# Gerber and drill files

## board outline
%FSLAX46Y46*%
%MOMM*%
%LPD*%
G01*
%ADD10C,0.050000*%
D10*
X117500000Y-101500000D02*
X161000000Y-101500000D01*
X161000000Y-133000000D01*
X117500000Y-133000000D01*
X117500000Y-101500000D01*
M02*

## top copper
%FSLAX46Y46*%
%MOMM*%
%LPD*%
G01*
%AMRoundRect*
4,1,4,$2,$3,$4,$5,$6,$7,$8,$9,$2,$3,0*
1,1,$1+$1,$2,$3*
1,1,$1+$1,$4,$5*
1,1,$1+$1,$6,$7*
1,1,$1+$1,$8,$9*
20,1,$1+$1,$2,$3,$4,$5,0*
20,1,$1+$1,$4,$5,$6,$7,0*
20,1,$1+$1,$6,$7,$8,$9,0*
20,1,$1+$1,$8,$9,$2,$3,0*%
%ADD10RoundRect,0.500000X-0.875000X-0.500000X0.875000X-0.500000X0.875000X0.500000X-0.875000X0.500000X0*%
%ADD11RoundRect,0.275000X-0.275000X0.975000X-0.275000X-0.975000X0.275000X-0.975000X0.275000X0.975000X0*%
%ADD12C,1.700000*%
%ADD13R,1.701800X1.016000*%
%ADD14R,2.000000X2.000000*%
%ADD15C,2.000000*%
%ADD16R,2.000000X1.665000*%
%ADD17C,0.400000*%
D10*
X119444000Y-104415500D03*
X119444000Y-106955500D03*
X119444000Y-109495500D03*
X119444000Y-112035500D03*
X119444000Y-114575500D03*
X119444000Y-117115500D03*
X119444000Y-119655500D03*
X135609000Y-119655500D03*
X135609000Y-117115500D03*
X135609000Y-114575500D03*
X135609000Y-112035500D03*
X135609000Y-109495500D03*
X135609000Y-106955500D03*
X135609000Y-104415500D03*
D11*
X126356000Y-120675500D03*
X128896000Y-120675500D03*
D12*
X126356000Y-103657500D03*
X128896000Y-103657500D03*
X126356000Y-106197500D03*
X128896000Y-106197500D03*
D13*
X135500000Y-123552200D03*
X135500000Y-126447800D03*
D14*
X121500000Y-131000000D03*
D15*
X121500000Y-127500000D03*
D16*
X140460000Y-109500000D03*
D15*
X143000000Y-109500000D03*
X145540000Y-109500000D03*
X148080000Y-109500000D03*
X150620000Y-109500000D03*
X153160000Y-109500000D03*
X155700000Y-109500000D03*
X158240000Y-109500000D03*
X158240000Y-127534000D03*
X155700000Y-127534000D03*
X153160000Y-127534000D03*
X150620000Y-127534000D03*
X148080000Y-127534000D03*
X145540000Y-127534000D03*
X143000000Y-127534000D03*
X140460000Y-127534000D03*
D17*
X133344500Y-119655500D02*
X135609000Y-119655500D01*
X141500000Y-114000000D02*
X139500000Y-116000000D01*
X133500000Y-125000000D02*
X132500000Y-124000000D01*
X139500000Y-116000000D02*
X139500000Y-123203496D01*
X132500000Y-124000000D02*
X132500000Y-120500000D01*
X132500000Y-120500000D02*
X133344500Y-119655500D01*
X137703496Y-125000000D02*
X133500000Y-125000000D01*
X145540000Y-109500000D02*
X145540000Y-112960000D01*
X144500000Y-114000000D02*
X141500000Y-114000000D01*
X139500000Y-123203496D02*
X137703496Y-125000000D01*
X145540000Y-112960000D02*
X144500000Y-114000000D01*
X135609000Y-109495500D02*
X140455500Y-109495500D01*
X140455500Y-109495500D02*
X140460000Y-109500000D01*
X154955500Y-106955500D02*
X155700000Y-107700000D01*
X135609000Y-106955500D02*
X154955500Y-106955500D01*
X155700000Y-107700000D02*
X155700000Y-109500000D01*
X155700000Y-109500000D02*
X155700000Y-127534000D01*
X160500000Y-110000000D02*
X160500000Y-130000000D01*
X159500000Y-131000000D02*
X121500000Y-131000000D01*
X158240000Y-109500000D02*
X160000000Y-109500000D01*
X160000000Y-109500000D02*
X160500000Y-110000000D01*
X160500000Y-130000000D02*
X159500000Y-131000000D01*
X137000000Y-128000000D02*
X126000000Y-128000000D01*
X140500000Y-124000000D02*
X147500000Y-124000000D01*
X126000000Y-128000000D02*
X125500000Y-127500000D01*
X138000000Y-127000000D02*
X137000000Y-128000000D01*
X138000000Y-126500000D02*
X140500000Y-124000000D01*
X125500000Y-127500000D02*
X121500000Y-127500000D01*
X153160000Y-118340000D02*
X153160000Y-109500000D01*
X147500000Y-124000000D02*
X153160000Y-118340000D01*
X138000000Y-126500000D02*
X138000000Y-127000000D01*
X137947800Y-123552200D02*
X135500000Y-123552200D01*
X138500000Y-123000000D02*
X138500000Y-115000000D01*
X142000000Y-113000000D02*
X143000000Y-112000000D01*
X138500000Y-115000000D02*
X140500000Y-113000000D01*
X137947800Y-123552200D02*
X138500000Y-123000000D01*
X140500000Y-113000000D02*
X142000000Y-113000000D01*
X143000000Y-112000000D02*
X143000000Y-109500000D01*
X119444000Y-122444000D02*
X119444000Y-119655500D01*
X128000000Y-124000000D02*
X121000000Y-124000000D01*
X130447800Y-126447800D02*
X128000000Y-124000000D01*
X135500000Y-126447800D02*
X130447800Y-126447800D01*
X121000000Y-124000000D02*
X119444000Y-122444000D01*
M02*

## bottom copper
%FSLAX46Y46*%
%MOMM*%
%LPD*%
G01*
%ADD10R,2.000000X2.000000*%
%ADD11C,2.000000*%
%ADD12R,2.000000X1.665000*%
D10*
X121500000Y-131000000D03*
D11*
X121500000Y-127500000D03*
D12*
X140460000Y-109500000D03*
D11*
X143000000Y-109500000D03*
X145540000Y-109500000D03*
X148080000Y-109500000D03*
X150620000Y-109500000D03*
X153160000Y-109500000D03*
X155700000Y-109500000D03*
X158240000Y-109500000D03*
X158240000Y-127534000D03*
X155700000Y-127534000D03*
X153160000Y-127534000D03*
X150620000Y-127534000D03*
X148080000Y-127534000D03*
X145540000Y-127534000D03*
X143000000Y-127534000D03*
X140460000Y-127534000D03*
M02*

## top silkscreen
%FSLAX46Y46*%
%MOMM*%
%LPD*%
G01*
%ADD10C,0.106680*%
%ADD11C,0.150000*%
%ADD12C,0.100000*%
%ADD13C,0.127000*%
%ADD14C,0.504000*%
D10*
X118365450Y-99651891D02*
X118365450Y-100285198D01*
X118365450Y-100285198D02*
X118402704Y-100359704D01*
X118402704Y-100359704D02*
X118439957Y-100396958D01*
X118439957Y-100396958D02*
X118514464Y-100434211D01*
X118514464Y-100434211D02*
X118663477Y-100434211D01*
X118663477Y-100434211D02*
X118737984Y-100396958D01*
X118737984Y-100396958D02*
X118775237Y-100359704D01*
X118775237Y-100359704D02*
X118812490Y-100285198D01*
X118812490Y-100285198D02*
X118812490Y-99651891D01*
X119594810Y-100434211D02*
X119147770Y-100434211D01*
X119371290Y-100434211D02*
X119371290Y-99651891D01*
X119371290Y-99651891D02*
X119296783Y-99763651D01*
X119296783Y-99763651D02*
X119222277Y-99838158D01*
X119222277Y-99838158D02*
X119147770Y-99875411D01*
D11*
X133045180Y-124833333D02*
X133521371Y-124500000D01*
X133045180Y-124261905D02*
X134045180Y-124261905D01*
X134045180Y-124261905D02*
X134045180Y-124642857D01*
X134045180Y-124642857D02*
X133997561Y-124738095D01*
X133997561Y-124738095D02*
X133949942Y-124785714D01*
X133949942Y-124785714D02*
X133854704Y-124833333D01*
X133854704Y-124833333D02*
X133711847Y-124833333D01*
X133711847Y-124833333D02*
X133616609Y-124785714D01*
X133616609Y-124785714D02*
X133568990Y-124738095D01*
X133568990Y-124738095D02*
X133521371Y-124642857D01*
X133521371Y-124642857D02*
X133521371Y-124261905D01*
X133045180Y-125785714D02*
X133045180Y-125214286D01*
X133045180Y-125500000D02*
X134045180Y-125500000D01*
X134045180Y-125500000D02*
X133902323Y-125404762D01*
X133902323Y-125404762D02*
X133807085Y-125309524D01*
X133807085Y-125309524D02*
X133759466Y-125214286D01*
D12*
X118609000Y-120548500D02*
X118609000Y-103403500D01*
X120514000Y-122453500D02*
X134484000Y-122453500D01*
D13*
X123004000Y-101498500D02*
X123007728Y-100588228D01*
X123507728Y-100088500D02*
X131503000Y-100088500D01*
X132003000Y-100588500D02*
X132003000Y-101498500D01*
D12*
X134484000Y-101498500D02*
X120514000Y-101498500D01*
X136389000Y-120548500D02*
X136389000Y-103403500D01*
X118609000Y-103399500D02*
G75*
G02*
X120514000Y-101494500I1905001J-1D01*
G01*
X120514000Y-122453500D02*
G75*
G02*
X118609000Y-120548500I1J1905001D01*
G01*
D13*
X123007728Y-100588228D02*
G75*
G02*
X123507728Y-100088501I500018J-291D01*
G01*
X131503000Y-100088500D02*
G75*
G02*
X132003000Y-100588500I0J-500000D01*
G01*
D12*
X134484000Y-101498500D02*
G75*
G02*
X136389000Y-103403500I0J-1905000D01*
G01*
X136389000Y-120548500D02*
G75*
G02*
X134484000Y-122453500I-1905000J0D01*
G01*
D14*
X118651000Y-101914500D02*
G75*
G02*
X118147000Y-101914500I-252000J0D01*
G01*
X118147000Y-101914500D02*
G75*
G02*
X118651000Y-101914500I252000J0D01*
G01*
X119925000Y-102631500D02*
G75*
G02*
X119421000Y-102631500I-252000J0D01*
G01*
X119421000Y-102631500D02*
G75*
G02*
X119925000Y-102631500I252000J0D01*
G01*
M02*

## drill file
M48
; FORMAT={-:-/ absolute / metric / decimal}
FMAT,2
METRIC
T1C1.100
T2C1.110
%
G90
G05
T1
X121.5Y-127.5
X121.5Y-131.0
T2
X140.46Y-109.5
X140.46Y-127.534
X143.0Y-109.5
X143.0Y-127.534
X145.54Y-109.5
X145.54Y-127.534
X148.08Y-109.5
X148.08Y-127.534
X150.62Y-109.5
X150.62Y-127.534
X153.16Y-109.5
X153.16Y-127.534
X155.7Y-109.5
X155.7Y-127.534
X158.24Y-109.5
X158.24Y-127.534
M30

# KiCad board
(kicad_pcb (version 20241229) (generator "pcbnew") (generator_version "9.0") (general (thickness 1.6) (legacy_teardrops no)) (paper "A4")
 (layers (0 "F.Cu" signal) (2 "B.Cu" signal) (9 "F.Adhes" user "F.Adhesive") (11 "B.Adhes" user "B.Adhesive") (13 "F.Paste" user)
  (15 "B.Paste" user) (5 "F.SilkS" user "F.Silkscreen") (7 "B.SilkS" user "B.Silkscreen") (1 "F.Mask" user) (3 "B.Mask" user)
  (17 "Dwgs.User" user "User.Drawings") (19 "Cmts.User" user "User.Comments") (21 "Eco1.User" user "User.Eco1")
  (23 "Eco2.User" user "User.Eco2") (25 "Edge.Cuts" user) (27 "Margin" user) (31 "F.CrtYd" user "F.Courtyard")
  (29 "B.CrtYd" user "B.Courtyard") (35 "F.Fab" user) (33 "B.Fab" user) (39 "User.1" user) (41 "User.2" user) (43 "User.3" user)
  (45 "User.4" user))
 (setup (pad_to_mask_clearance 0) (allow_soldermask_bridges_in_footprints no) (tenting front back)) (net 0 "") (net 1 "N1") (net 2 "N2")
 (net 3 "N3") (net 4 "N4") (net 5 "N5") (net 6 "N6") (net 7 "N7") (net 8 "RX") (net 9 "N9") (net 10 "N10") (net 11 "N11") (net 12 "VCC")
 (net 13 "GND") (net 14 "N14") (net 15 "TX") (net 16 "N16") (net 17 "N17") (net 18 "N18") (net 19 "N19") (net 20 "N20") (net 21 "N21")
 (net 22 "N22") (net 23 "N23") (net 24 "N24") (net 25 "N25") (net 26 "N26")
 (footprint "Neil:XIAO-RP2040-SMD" (layer "F.Cu") (at 127.444 112.0355)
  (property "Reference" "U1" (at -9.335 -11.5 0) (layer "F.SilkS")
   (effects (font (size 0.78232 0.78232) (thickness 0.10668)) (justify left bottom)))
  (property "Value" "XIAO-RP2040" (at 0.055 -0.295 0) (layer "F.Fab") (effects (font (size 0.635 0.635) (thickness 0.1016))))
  (fp_line (start -8.835 8.513) (end -8.835 -8.632) (stroke (width 0.1) (type solid)) (layer "F.SilkS"))
  (fp_line (start -6.93 10.418) (end 7.04 10.418) (stroke (width 0.1) (type solid)) (layer "F.SilkS"))
  (fp_line (start -4.44 -10.537) (end -4.436272 -11.447272) (stroke (width 0.127) (type solid)) (layer "F.SilkS"))
  (fp_line (start -3.936272 -11.947) (end 4.059 -11.947) (stroke (width 0.127) (type solid)) (layer "F.SilkS"))
  (fp_line (start 4.559 -11.447) (end 4.559 -10.537) (stroke (width 0.127) (type solid)) (layer "F.SilkS"))
  (fp_line (start 7.04 -10.537) (end -6.93 -10.537) (stroke (width 0.1) (type solid)) (layer "F.SilkS"))
  (fp_line (start 8.945 8.513) (end 8.945 -8.632) (stroke (width 0.1) (type solid)) (layer "F.SilkS"))
  (fp_arc (start -8.835 -8.636) (mid -8.277038 -9.983038) (end -6.93 -10.541) (stroke (width 0.1) (type solid)) (layer "F.SilkS"))
  (fp_arc (start -6.93 10.418) (mid -8.277038 9.860038) (end -8.835 8.513) (stroke (width 0.1) (type solid)) (layer "F.SilkS"))
  (fp_arc (start -4.436272 -11.447272) (mid -4.289724 -11.800644) (end -3.936272 -11.947) (stroke (width 0.127) (type default))
   (layer "F.SilkS"))
  (fp_arc (start 4.059 -11.947) (mid 4.412553 -11.800553) (end 4.559 -11.447) (stroke (width 0.127) (type default)) (layer "F.SilkS"))
  (fp_arc (start 7.04 -10.537) (mid 8.387038 -9.979038) (end 8.945 -8.632) (stroke (width 0.1) (type solid)) (layer "F.SilkS"))
  (fp_arc (start 8.945 8.513) (mid 8.387038 9.860038) (end 7.04 10.418) (stroke (width 0.1) (type solid)) (layer "F.SilkS"))
  (fp_circle (center -9.045 -10.121) (end -9.045 -10.375) (stroke (width 0.5) (type solid)) (fill yes) (layer "F.SilkS"))
  (fp_circle (center -7.771 -9.404) (end -7.771 -9.658) (stroke (width 0.5) (type solid)) (fill yes) (layer "F.SilkS"))
  (pad "1" smd roundrect (at -8 -7.62) (size 2.75 2) (layers "F.Cu" "F.Mask" "F.Paste") (roundrect_rratio 0.25) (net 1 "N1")
   (solder_mask_margin 0.0508) (thermal_bridge_angle 45))
  (pad "2" smd roundrect (at -8 -5.08) (size 2.75 2) (layers "F.Cu" "F.Mask" "F.Paste") (roundrect_rratio 0.25) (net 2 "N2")
   (solder_mask_margin 0.0508) (thermal_bridge_angle 45))
  (pad "3" smd roundrect (at -8 -2.54) (size 2.75 2) (layers "F.Cu" "F.Mask" "F.Paste") (roundrect_rratio 0.25) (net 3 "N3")
   (solder_mask_margin 0.0508) (thermal_bridge_angle 45))
  (pad "4" smd roundrect (at -8 0) (size 2.75 2) (layers "F.Cu" "F.Mask" "F.Paste") (roundrect_rratio 0.25) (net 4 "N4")
   (solder_mask_margin 0.0508) (thermal_bridge_angle 45))
  (pad "5" smd roundrect (at -8 2.54) (size 2.75 2) (layers "F.Cu" "F.Mask" "F.Paste") (roundrect_rratio 0.25) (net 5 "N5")
   (solder_mask_margin 0.0508) (thermal_bridge_angle 45))
  (pad "6" smd roundrect (at -8 5.08) (size 2.75 2) (layers "F.Cu" "F.Mask" "F.Paste") (roundrect_rratio 0.25) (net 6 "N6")
   (solder_mask_margin 0.0508) (thermal_bridge_angle 45))
  (pad "7" smd roundrect (at -8 7.62) (size 2.75 2) (layers "F.Cu" "F.Mask" "F.Paste") (roundrect_rratio 0.25) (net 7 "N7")
   (solder_mask_margin 0.0508) (thermal_bridge_angle 45))
  (pad "8" smd roundrect (at 8.165 7.62) (size 2.75 2) (layers "F.Cu" "F.Mask" "F.Paste") (roundrect_rratio 0.25) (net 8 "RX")
   (solder_mask_margin 0.0508) (thermal_bridge_angle 45))
  (pad "9" smd roundrect (at 8.165 5.08) (size 2.75 2) (layers "F.Cu" "F.Mask" "F.Paste") (roundrect_rratio 0.25) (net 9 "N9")
   (solder_mask_margin 0.0508) (thermal_bridge_angle 45))
  (pad "10" smd roundrect (at 8.165 2.54) (size 2.75 2) (layers "F.Cu" "F.Mask" "F.Paste") (roundrect_rratio 0.25) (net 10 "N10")
   (solder_mask_margin 0.0508) (thermal_bridge_angle 45))
  (pad "11" smd roundrect (at 8.165 0) (size 2.75 2) (layers "F.Cu" "F.Mask" "F.Paste") (roundrect_rratio 0.25) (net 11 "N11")
   (solder_mask_margin 0.0508) (thermal_bridge_angle 45))
  (pad "12" smd roundrect (at 8.165 -2.54) (size 2.75 2) (layers "F.Cu" "F.Mask" "F.Paste") (roundrect_rratio 0.25) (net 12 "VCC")
   (solder_mask_margin 0.0508) (thermal_bridge_angle 45))
  (pad "13" smd roundrect (at 8.165 -5.08) (size 2.75 2) (layers "F.Cu" "F.Mask" "F.Paste") (roundrect_rratio 0.25) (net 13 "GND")
   (solder_mask_margin 0.0508) (thermal_bridge_angle 45))
  (pad "14" smd roundrect (at 8.165 -7.62) (size 2.75 2) (layers "F.Cu" "F.Mask" "F.Paste") (roundrect_rratio 0.25) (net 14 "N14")
   (solder_mask_margin 0.0508) (thermal_bridge_angle 45))
  (pad "15" smd roundrect (at -1.088 8.64 270) (size 2.5 1.1) (layers "F.Cu" "F.Mask" "F.Paste") (roundrect_rratio 0.25)
   (thermal_bridge_angle 45))
  (pad "16" smd roundrect (at 1.452 8.64 270) (size 2.5 1.1) (layers "F.Cu" "F.Mask" "F.Paste") (roundrect_rratio 0.25)
   (thermal_bridge_angle 45))
  (pad "17" smd circle (at -1.088 -8.378) (size 1.7 1.7) (layers "F.Cu" "F.Mask" "F.Paste"))
  (pad "18" smd circle (at 1.452 -8.378) (size 1.7 1.7) (layers "F.Cu" "F.Mask" "F.Paste"))
  (pad "19" smd circle (at -1.088 -5.838) (size 1.7 1.7) (layers "F.Cu" "F.Mask" "F.Paste"))
  (pad "20" smd circle (at 1.452 -5.838) (size 1.7 1.7) (layers "F.Cu" "F.Mask" "F.Paste")))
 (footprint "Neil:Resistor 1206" (layer "F.Cu") (at 135.5 125 -90)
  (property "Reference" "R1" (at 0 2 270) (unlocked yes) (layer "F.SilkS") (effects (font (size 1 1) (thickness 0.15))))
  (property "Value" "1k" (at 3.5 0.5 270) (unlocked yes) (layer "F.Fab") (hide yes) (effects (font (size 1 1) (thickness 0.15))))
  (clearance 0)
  (pad "1" smd rect (at -1.4478 0 270) (size 1.016 1.7018) (layers "F.Cu" "F.Mask" "F.Paste") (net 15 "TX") (clearance -1))
  (pad "2" smd rect (at 1.4478 0 270) (size 1.016 1.7018) (layers "F.Cu" "F.Mask" "F.Paste") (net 7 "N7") (clearance -1)))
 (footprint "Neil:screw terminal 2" (layer "B.Cu") (at 121.5 131 90)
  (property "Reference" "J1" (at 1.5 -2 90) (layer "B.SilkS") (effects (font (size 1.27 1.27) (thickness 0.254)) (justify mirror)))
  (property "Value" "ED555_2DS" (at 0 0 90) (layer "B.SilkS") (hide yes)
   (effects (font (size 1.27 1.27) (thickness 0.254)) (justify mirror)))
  (pad "1" thru_hole rect (at 0 0 90) (size 2 2) (drill 1.1) (layers "*.Cu" "*.Mask") (remove_unused_layers no) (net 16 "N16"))
  (pad "2" thru_hole circle (at 3.5 0 90) (size 2 2) (drill 1.1) (layers "*.Cu" "*.Mask") (remove_unused_layers no) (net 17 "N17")))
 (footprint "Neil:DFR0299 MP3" (layer "B.Cu") (at 140.46 109.5)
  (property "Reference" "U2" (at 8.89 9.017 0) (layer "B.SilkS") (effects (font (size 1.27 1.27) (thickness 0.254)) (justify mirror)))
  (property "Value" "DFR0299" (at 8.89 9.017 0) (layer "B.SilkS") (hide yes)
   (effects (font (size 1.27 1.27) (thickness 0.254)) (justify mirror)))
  (pad "1" thru_hole rect (at 0 0) (size 2 1.665) (drill 1.11) (layers "*.Cu" "*.Mask") (remove_unused_layers no) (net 12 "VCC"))
  (pad "2" thru_hole circle (at 2.54 0) (size 2 2) (drill 1.11) (layers "*.Cu" "*.Mask") (remove_unused_layers no) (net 15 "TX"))
  (pad "3" thru_hole circle (at 5.08 0) (size 2 2) (drill 1.11) (layers "*.Cu" "*.Mask") (remove_unused_layers no) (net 8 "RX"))
  (pad "4" thru_hole circle (at 7.62 0) (size 2 2) (drill 1.11) (layers "*.Cu" "*.Mask") (remove_unused_layers no) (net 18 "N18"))
  (pad "5" thru_hole circle (at 10.16 0) (size 2 2) (drill 1.11) (layers "*.Cu" "*.Mask") (remove_unused_layers no) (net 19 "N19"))
  (pad "6" thru_hole circle (at 12.7 0) (size 2 2) (drill 1.11) (layers "*.Cu" "*.Mask") (remove_unused_layers no) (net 17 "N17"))
  (pad "7" thru_hole circle (at 15.24 0) (size 2 2) (drill 1.11) (layers "*.Cu" "*.Mask") (remove_unused_layers no) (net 13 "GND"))
  (pad "8" thru_hole circle (at 17.78 0) (size 2 2) (drill 1.11) (layers "*.Cu" "*.Mask") (remove_unused_layers no) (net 16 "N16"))
  (pad "9" thru_hole circle (at 17.78 18.034) (size 2 2) (drill 1.11) (layers "*.Cu" "*.Mask") (remove_unused_layers no) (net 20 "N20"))
  (pad "10" thru_hole circle (at 15.24 18.034) (size 2 2) (drill 1.11) (layers "*.Cu" "*.Mask") (remove_unused_layers no) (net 13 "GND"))
  (pad "11" thru_hole circle (at 12.7 18.034) (size 2 2) (drill 1.11) (layers "*.Cu" "*.Mask") (remove_unused_layers no) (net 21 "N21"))
  (pad "12" thru_hole circle (at 10.16 18.034) (size 2 2) (drill 1.11) (layers "*.Cu" "*.Mask") (remove_unused_layers no) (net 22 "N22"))
  (pad "13" thru_hole circle (at 7.62 18.034) (size 2 2) (drill 1.11) (layers "*.Cu" "*.Mask") (remove_unused_layers no) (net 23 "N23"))
  (pad "14" thru_hole circle (at 5.08 18.034) (size 2 2) (drill 1.11) (layers "*.Cu" "*.Mask") (remove_unused_layers no) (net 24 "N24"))
  (pad "15" thru_hole circle (at 2.54 18.034) (size 2 2) (drill 1.11) (layers "*.Cu" "*.Mask") (remove_unused_layers no) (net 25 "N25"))
  (pad "16" thru_hole circle (at 0 18.034) (size 2 2) (drill 1.11) (layers "*.Cu" "*.Mask") (remove_unused_layers no) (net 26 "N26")))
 (gr_rect (start 117.5 101.5) (end 161 133) (stroke (width 0.05) (type default)) (fill no) (layer "Edge.Cuts"))
 (segment (start 133.3445 119.6555) (end 135.609 119.6555) (width 0.4) (layer "F.Cu") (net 8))
 (segment (start 141.5 114) (end 139.5 116) (width 0.4) (layer "F.Cu") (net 8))
 (segment (start 133.5 125) (end 132.5 124) (width 0.4) (layer "F.Cu") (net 8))
 (segment (start 139.5 116) (end 139.5 123.203496) (width 0.4) (layer "F.Cu") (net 8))
 (segment (start 132.5 124) (end 132.5 120.5) (width 0.4) (layer "F.Cu") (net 8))
 (segment (start 132.5 120.5) (end 133.3445 119.6555) (width 0.4) (layer "F.Cu") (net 8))
 (segment (start 137.703496 125) (end 133.5 125) (width 0.4) (layer "F.Cu") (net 8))
 (segment (start 145.54 109.5) (end 145.54 112.96) (width 0.4) (layer "F.Cu") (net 8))
 (segment (start 144.5 114) (end 141.5 114) (width 0.4) (layer "F.Cu") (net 8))
 (segment (start 139.5 123.203496) (end 137.703496 125) (width 0.4) (layer "F.Cu") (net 8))
 (segment (start 145.54 112.96) (end 144.5 114) (width 0.4) (layer "F.Cu") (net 8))
 (segment (start 135.609 109.4955) (end 140.4555 109.4955) (width 0.4) (layer "F.Cu") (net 12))
 (segment (start 140.4555 109.4955) (end 140.46 109.5) (width 0.4) (layer "F.Cu") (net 12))
 (segment (start 154.9555 106.9555) (end 155.7 107.7) (width 0.4) (layer "F.Cu") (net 13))
 (segment (start 135.609 106.9555) (end 154.9555 106.9555) (width 0.4) (layer "F.Cu") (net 13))
 (segment (start 155.7 107.7) (end 155.7 109.5) (width 0.4) (layer "F.Cu") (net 13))
 (segment (start 155.7 109.5) (end 155.7 127.534) (width 0.4) (layer "F.Cu") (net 13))
 (segment (start 160.5 110) (end 160.5 130) (width 0.4) (layer "F.Cu") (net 16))
 (segment (start 159.5 131) (end 121.5 131) (width 0.4) (layer "F.Cu") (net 16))
 (segment (start 158.24 109.5) (end 160 109.5) (width 0.4) (layer "F.Cu") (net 16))
 (segment (start 160 109.5) (end 160.5 110) (width 0.4) (layer "F.Cu") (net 16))
 (segment (start 160.5 130) (end 159.5 131) (width 0.4) (layer "F.Cu") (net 16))
 (segment (start 137 128) (end 126 128) (width 0.4) (layer "F.Cu") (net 17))
 (segment (start 140.5 124) (end 147.5 124) (width 0.4) (layer "F.Cu") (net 17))
 (segment (start 126 128) (end 125.5 127.5) (width 0.4) (layer "F.Cu") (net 17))
 (segment (start 138 127) (end 137 128) (width 0.4) (layer "F.Cu") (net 17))
 (segment (start 138 126.5) (end 140.5 124) (width 0.4) (layer "F.Cu") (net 17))
 (segment (start 125.5 127.5) (end 121.5 127.5) (width 0.4) (layer "F.Cu") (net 17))
 (segment (start 153.16 118.34) (end 153.16 109.5) (width 0.4) (layer "F.Cu") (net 17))
 (segment (start 147.5 124) (end 153.16 118.34) (width 0.4) (layer "F.Cu") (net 17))
 (segment (start 138 126.5) (end 138 127) (width 0.4) (layer "F.Cu") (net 17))
 (segment (start 137.9478 123.5522) (end 135.5 123.5522) (width 0.4) (layer "F.Cu") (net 15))
 (segment (start 138.5 123) (end 138.5 115) (width 0.4) (layer "F.Cu") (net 15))
 (segment (start 142 113) (end 143 112) (width 0.4) (layer "F.Cu") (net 15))
 (segment (start 138.5 115) (end 140.5 113) (width 0.4) (layer "F.Cu") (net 15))
 (segment (start 137.9478 123.5522) (end 138.5 123) (width 0.4) (layer "F.Cu") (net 15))
 (segment (start 140.5 113) (end 142 113) (width 0.4) (layer "F.Cu") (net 15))
 (segment (start 143 112) (end 143 109.5) (width 0.4) (layer "F.Cu") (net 15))
 (segment (start 119.444 122.444) (end 119.444 119.6555) (width 0.4) (layer "F.Cu") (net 7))
 (segment (start 128 124) (end 121 124) (width 0.4) (layer "F.Cu") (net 7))
 (segment (start 130.4478 126.4478) (end 128 124) (width 0.4) (layer "F.Cu") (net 7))
 (segment (start 135.5 126.4478) (end 130.4478 126.4478) (width 0.4) (layer "F.Cu") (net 7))
 (segment (start 121 124) (end 119.444 122.444) (width 0.4) (layer "F.Cu") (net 7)))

